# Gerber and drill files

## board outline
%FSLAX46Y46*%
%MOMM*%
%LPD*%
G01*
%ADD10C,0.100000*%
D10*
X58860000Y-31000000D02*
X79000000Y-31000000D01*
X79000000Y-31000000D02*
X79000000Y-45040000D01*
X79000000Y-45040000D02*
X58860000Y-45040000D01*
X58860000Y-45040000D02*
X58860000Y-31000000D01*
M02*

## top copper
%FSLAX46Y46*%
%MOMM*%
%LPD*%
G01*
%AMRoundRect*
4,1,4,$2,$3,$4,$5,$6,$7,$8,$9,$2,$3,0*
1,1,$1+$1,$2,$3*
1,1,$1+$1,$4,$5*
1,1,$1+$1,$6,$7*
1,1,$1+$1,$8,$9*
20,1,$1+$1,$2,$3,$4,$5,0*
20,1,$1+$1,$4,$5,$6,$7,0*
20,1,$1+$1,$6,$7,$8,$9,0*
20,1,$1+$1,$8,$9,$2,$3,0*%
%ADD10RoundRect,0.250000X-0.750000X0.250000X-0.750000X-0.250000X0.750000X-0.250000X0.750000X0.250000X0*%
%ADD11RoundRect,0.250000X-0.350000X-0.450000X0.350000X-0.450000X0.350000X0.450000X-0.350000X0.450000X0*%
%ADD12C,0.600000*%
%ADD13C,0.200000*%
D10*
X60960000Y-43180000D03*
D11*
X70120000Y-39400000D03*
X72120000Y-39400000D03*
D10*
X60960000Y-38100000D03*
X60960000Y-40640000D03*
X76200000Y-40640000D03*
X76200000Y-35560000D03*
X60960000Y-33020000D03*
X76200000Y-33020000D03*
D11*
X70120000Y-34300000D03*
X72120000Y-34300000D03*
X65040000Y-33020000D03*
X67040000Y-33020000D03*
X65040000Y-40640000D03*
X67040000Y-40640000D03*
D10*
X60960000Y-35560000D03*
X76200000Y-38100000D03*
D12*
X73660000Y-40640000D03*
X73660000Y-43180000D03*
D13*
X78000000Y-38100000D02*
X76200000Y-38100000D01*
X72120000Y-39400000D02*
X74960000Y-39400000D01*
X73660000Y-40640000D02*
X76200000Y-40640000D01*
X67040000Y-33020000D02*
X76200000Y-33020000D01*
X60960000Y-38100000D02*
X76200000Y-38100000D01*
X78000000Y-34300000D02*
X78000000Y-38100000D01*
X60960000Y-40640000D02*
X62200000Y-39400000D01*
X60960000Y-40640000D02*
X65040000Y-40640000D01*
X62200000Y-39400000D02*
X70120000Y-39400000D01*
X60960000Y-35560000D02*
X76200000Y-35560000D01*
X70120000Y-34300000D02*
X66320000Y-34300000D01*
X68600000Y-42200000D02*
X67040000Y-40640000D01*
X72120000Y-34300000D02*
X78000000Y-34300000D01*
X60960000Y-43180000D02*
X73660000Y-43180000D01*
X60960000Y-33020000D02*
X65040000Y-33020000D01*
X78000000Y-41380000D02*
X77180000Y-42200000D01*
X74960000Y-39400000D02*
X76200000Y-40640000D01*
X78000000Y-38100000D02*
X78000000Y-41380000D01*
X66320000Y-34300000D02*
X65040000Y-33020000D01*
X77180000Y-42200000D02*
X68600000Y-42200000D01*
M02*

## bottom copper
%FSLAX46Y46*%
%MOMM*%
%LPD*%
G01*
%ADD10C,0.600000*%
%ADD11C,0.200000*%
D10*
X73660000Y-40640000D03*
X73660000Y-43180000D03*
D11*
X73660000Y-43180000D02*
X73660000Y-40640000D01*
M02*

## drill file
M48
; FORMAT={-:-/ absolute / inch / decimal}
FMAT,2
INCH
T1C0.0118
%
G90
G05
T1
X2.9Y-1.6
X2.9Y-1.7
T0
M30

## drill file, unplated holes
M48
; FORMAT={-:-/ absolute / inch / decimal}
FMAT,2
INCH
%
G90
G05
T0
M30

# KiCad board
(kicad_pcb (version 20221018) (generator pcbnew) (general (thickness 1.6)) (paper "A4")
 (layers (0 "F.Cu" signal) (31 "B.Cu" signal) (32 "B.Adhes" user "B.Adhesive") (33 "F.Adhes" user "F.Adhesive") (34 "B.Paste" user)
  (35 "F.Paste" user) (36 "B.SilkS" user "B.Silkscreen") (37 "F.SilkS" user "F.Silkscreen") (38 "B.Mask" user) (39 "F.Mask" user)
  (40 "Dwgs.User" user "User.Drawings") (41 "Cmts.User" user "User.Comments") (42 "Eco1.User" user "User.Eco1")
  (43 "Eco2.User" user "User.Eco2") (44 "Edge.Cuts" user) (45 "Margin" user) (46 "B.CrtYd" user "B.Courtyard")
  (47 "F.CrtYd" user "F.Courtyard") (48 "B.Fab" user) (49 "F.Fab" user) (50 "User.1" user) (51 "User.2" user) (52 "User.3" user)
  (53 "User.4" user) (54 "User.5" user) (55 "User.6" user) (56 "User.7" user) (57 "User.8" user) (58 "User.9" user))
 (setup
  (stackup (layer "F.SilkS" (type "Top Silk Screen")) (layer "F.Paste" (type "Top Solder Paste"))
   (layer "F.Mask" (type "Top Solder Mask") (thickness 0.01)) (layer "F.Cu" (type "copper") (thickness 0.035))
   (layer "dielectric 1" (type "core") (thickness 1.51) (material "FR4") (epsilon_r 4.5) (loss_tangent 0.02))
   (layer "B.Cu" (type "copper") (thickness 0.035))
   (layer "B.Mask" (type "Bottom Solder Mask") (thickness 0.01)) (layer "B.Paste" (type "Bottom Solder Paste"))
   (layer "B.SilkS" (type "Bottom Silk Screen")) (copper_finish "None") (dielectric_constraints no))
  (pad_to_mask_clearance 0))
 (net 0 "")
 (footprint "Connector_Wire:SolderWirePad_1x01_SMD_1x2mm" (layer "F.Cu") (at 60.96 43.18 -90)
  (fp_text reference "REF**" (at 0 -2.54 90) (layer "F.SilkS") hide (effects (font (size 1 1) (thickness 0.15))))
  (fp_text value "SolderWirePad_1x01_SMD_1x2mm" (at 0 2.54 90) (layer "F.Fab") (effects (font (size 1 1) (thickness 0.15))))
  (pad "5" smd roundrect (at 0 0 270) (size 1 2) (layers "F.Cu" "F.Paste" "F.Mask") (roundrect_rratio 0.25)))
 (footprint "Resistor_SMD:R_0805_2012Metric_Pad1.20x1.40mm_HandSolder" (layer "F.Cu") (at 71.12 39.4)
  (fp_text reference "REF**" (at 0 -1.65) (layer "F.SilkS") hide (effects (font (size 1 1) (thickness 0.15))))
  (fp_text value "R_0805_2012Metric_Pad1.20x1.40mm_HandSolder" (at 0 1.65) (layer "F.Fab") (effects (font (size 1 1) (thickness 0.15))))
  (pad "1" smd roundrect (at -1 0) (size 1.2 1.4) (layers "F.Cu" "F.Paste" "F.Mask") (roundrect_rratio 0.2083333333))
  (pad "2" smd roundrect (at 1 0) (size 1.2 1.4) (layers "F.Cu" "F.Paste" "F.Mask") (roundrect_rratio 0.2083333333)))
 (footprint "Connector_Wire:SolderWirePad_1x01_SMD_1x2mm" (layer "F.Cu") (at 60.96 38.1 -90)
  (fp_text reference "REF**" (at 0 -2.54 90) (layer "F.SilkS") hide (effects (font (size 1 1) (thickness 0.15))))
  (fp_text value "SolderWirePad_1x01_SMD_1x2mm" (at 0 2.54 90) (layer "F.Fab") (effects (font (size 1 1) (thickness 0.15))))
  (pad "3" smd roundrect (at 0 0 270) (size 1 2) (layers "F.Cu" "F.Paste" "F.Mask") (roundrect_rratio 0.25)))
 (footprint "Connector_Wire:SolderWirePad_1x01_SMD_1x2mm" (layer "F.Cu") (at 60.96 40.64 -90)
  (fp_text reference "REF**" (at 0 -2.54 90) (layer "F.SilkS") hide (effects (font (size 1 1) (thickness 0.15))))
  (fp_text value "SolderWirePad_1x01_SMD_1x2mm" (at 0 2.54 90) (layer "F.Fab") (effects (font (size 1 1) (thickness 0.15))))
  (pad "4" smd roundrect (at 0 0 270) (size 1 2) (layers "F.Cu" "F.Paste" "F.Mask") (roundrect_rratio 0.25)))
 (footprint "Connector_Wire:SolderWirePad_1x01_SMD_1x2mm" (layer "F.Cu") (at 76.2 40.64 -90)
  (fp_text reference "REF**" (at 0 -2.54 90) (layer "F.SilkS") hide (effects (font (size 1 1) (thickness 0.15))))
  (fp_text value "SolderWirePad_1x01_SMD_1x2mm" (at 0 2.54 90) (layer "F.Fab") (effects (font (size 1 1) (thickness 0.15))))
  (pad "9" smd roundrect (at 0 0 270) (size 1 2) (layers "F.Cu" "F.Paste" "F.Mask") (roundrect_rratio 0.25)))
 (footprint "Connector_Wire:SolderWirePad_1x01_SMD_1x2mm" (layer "F.Cu") (at 76.2 35.56 -90)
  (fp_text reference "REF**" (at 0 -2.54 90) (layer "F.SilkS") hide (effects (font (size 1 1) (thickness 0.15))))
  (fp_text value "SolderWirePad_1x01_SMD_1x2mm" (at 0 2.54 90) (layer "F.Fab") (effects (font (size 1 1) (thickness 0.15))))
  (pad "7" smd roundrect (at 0 0 270) (size 1 2) (layers "F.Cu" "F.Paste" "F.Mask") (roundrect_rratio 0.25)))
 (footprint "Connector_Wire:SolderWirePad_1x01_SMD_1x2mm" (layer "F.Cu") (at 60.96 33.02 -90)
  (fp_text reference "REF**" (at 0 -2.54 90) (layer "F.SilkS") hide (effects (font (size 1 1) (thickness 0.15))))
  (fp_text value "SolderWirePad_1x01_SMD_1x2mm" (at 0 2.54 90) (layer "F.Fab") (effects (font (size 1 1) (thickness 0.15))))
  (pad "1" smd roundrect (at 0 0 270) (size 1 2) (layers "F.Cu" "F.Paste" "F.Mask") (roundrect_rratio 0.25)))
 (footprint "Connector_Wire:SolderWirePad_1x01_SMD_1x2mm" (layer "F.Cu") (at 76.2 33.02 -90)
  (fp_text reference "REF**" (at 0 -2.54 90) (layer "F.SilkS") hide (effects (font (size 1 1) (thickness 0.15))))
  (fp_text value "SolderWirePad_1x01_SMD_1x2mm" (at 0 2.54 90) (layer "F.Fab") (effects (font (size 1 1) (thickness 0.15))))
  (pad "6" smd roundrect (at 0 0 270) (size 1 2) (layers "F.Cu" "F.Paste" "F.Mask") (roundrect_rratio 0.25)))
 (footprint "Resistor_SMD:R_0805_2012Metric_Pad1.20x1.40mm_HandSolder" (layer "F.Cu") (at 71.12 34.3)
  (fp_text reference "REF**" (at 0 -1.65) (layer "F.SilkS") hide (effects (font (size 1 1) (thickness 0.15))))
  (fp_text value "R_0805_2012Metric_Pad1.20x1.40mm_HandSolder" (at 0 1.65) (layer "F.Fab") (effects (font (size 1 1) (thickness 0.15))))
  (pad "1" smd roundrect (at -1 0) (size 1.2 1.4) (layers "F.Cu" "F.Paste" "F.Mask") (roundrect_rratio 0.2083333333))
  (pad "2" smd roundrect (at 1 0) (size 1.2 1.4) (layers "F.Cu" "F.Paste" "F.Mask") (roundrect_rratio 0.2083333333)))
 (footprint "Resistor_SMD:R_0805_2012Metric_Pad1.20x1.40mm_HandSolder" (layer "F.Cu") (at 66.04 33.02)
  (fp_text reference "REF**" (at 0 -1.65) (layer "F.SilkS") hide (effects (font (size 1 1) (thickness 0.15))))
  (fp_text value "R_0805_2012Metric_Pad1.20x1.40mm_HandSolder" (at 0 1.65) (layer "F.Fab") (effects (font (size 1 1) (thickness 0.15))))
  (pad "1" smd roundrect (at -1 0) (size 1.2 1.4) (layers "F.Cu" "F.Paste" "F.Mask") (roundrect_rratio 0.2083333333))
  (pad "2" smd roundrect (at 1 0) (size 1.2 1.4) (layers "F.Cu" "F.Paste" "F.Mask") (roundrect_rratio 0.2083333333)))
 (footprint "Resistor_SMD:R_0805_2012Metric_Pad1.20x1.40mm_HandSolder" (layer "F.Cu") (at 66.04 40.64)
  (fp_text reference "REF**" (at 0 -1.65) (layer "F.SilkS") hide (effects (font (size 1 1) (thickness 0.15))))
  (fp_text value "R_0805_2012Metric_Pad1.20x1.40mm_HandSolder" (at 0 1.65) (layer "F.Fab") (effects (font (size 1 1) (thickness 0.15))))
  (pad "1" smd roundrect (at -1 0) (size 1.2 1.4) (layers "F.Cu" "F.Paste" "F.Mask") (roundrect_rratio 0.2083333333))
  (pad "2" smd roundrect (at 1 0) (size 1.2 1.4) (layers "F.Cu" "F.Paste" "F.Mask") (roundrect_rratio 0.2083333333)))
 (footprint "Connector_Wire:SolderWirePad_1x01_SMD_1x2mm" (layer "F.Cu") (at 60.96 35.56 -90)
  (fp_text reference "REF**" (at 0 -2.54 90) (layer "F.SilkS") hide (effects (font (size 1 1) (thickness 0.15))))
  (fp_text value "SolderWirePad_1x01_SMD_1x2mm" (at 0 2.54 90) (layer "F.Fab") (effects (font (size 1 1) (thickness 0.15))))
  (pad "2" smd roundrect (at 0 0 270) (size 1 2) (layers "F.Cu" "F.Paste" "F.Mask") (roundrect_rratio 0.25)))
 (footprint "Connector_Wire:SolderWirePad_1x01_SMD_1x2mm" (layer "F.Cu") (at 76.2 38.1 -90)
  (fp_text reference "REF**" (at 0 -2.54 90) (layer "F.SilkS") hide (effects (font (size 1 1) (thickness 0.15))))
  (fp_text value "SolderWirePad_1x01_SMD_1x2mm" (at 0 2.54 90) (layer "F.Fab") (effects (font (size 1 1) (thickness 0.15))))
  (pad "8" smd roundrect (at 0 0 270) (size 1 2) (layers "F.Cu" "F.Paste" "F.Mask") (roundrect_rratio 0.25)))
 (gr_rect (start 58.86 31) (end 79 45.04) (stroke (width 0.1) (type default)) (fill none) (layer "Edge.Cuts"))
 (segment (start 78 38.1) (end 76.2 38.1) (width 0.2) (layer "F.Cu") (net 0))
 (segment (start 72.12 39.4) (end 74.96 39.4) (width 0.2) (layer "F.Cu") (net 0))
 (segment (start 73.66 40.64) (end 76.2 40.64) (width 0.2) (layer "F.Cu") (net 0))
 (segment (start 67.04 33.02) (end 76.2 33.02) (width 0.2) (layer "F.Cu") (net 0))
 (segment (start 60.96 38.1) (end 76.2 38.1) (width 0.2) (layer "F.Cu") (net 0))
 (segment (start 78 34.3) (end 78 38.1) (width 0.2) (layer "F.Cu") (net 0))
 (segment (start 60.96 40.64) (end 62.2 39.4) (width 0.2) (layer "F.Cu") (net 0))
 (segment (start 60.96 40.64) (end 65.04 40.64) (width 0.2) (layer "F.Cu") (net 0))
 (segment (start 62.2 39.4) (end 70.12 39.4) (width 0.2) (layer "F.Cu") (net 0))
 (segment (start 60.96 35.56) (end 76.2 35.56) (width 0.2) (layer "F.Cu") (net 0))
 (segment (start 70.12 34.3) (end 66.32 34.3) (width 0.2) (layer "F.Cu") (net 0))
 (segment (start 68.6 42.2) (end 67.04 40.64) (width 0.2) (layer "F.Cu") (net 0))
 (segment (start 72.12 34.3) (end 78 34.3) (width 0.2) (layer "F.Cu") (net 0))
 (segment (start 60.96 43.18) (end 73.66 43.18) (width 0.2) (layer "F.Cu") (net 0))
 (segment (start 60.96 33.02) (end 65.04 33.02) (width 0.2) (layer "F.Cu") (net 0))
 (segment (start 78 41.38) (end 77.18 42.2) (width 0.2) (layer "F.Cu") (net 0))
 (segment (start 74.96 39.4) (end 76.2 40.64) (width 0.2) (layer "F.Cu") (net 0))
 (segment (start 78 38.1) (end 78 41.38) (width 0.2) (layer "F.Cu") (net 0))
 (segment (start 66.32 34.3) (end 65.04 33.02) (width 0.2) (layer "F.Cu") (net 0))
 (segment (start 77.18 42.2) (end 68.6 42.2) (width 0.2) (layer "F.Cu") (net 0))
 (via (at 73.66 40.64) (size 0.6) (drill 0.3) (layers "F.Cu" "B.Cu") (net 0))
 (via (at 73.66 43.18) (size 0.6) (drill 0.3) (layers "F.Cu" "B.Cu") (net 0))
 (segment (start 73.66 43.18) (end 73.66 40.64) (width 0.2) (layer "B.Cu") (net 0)))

